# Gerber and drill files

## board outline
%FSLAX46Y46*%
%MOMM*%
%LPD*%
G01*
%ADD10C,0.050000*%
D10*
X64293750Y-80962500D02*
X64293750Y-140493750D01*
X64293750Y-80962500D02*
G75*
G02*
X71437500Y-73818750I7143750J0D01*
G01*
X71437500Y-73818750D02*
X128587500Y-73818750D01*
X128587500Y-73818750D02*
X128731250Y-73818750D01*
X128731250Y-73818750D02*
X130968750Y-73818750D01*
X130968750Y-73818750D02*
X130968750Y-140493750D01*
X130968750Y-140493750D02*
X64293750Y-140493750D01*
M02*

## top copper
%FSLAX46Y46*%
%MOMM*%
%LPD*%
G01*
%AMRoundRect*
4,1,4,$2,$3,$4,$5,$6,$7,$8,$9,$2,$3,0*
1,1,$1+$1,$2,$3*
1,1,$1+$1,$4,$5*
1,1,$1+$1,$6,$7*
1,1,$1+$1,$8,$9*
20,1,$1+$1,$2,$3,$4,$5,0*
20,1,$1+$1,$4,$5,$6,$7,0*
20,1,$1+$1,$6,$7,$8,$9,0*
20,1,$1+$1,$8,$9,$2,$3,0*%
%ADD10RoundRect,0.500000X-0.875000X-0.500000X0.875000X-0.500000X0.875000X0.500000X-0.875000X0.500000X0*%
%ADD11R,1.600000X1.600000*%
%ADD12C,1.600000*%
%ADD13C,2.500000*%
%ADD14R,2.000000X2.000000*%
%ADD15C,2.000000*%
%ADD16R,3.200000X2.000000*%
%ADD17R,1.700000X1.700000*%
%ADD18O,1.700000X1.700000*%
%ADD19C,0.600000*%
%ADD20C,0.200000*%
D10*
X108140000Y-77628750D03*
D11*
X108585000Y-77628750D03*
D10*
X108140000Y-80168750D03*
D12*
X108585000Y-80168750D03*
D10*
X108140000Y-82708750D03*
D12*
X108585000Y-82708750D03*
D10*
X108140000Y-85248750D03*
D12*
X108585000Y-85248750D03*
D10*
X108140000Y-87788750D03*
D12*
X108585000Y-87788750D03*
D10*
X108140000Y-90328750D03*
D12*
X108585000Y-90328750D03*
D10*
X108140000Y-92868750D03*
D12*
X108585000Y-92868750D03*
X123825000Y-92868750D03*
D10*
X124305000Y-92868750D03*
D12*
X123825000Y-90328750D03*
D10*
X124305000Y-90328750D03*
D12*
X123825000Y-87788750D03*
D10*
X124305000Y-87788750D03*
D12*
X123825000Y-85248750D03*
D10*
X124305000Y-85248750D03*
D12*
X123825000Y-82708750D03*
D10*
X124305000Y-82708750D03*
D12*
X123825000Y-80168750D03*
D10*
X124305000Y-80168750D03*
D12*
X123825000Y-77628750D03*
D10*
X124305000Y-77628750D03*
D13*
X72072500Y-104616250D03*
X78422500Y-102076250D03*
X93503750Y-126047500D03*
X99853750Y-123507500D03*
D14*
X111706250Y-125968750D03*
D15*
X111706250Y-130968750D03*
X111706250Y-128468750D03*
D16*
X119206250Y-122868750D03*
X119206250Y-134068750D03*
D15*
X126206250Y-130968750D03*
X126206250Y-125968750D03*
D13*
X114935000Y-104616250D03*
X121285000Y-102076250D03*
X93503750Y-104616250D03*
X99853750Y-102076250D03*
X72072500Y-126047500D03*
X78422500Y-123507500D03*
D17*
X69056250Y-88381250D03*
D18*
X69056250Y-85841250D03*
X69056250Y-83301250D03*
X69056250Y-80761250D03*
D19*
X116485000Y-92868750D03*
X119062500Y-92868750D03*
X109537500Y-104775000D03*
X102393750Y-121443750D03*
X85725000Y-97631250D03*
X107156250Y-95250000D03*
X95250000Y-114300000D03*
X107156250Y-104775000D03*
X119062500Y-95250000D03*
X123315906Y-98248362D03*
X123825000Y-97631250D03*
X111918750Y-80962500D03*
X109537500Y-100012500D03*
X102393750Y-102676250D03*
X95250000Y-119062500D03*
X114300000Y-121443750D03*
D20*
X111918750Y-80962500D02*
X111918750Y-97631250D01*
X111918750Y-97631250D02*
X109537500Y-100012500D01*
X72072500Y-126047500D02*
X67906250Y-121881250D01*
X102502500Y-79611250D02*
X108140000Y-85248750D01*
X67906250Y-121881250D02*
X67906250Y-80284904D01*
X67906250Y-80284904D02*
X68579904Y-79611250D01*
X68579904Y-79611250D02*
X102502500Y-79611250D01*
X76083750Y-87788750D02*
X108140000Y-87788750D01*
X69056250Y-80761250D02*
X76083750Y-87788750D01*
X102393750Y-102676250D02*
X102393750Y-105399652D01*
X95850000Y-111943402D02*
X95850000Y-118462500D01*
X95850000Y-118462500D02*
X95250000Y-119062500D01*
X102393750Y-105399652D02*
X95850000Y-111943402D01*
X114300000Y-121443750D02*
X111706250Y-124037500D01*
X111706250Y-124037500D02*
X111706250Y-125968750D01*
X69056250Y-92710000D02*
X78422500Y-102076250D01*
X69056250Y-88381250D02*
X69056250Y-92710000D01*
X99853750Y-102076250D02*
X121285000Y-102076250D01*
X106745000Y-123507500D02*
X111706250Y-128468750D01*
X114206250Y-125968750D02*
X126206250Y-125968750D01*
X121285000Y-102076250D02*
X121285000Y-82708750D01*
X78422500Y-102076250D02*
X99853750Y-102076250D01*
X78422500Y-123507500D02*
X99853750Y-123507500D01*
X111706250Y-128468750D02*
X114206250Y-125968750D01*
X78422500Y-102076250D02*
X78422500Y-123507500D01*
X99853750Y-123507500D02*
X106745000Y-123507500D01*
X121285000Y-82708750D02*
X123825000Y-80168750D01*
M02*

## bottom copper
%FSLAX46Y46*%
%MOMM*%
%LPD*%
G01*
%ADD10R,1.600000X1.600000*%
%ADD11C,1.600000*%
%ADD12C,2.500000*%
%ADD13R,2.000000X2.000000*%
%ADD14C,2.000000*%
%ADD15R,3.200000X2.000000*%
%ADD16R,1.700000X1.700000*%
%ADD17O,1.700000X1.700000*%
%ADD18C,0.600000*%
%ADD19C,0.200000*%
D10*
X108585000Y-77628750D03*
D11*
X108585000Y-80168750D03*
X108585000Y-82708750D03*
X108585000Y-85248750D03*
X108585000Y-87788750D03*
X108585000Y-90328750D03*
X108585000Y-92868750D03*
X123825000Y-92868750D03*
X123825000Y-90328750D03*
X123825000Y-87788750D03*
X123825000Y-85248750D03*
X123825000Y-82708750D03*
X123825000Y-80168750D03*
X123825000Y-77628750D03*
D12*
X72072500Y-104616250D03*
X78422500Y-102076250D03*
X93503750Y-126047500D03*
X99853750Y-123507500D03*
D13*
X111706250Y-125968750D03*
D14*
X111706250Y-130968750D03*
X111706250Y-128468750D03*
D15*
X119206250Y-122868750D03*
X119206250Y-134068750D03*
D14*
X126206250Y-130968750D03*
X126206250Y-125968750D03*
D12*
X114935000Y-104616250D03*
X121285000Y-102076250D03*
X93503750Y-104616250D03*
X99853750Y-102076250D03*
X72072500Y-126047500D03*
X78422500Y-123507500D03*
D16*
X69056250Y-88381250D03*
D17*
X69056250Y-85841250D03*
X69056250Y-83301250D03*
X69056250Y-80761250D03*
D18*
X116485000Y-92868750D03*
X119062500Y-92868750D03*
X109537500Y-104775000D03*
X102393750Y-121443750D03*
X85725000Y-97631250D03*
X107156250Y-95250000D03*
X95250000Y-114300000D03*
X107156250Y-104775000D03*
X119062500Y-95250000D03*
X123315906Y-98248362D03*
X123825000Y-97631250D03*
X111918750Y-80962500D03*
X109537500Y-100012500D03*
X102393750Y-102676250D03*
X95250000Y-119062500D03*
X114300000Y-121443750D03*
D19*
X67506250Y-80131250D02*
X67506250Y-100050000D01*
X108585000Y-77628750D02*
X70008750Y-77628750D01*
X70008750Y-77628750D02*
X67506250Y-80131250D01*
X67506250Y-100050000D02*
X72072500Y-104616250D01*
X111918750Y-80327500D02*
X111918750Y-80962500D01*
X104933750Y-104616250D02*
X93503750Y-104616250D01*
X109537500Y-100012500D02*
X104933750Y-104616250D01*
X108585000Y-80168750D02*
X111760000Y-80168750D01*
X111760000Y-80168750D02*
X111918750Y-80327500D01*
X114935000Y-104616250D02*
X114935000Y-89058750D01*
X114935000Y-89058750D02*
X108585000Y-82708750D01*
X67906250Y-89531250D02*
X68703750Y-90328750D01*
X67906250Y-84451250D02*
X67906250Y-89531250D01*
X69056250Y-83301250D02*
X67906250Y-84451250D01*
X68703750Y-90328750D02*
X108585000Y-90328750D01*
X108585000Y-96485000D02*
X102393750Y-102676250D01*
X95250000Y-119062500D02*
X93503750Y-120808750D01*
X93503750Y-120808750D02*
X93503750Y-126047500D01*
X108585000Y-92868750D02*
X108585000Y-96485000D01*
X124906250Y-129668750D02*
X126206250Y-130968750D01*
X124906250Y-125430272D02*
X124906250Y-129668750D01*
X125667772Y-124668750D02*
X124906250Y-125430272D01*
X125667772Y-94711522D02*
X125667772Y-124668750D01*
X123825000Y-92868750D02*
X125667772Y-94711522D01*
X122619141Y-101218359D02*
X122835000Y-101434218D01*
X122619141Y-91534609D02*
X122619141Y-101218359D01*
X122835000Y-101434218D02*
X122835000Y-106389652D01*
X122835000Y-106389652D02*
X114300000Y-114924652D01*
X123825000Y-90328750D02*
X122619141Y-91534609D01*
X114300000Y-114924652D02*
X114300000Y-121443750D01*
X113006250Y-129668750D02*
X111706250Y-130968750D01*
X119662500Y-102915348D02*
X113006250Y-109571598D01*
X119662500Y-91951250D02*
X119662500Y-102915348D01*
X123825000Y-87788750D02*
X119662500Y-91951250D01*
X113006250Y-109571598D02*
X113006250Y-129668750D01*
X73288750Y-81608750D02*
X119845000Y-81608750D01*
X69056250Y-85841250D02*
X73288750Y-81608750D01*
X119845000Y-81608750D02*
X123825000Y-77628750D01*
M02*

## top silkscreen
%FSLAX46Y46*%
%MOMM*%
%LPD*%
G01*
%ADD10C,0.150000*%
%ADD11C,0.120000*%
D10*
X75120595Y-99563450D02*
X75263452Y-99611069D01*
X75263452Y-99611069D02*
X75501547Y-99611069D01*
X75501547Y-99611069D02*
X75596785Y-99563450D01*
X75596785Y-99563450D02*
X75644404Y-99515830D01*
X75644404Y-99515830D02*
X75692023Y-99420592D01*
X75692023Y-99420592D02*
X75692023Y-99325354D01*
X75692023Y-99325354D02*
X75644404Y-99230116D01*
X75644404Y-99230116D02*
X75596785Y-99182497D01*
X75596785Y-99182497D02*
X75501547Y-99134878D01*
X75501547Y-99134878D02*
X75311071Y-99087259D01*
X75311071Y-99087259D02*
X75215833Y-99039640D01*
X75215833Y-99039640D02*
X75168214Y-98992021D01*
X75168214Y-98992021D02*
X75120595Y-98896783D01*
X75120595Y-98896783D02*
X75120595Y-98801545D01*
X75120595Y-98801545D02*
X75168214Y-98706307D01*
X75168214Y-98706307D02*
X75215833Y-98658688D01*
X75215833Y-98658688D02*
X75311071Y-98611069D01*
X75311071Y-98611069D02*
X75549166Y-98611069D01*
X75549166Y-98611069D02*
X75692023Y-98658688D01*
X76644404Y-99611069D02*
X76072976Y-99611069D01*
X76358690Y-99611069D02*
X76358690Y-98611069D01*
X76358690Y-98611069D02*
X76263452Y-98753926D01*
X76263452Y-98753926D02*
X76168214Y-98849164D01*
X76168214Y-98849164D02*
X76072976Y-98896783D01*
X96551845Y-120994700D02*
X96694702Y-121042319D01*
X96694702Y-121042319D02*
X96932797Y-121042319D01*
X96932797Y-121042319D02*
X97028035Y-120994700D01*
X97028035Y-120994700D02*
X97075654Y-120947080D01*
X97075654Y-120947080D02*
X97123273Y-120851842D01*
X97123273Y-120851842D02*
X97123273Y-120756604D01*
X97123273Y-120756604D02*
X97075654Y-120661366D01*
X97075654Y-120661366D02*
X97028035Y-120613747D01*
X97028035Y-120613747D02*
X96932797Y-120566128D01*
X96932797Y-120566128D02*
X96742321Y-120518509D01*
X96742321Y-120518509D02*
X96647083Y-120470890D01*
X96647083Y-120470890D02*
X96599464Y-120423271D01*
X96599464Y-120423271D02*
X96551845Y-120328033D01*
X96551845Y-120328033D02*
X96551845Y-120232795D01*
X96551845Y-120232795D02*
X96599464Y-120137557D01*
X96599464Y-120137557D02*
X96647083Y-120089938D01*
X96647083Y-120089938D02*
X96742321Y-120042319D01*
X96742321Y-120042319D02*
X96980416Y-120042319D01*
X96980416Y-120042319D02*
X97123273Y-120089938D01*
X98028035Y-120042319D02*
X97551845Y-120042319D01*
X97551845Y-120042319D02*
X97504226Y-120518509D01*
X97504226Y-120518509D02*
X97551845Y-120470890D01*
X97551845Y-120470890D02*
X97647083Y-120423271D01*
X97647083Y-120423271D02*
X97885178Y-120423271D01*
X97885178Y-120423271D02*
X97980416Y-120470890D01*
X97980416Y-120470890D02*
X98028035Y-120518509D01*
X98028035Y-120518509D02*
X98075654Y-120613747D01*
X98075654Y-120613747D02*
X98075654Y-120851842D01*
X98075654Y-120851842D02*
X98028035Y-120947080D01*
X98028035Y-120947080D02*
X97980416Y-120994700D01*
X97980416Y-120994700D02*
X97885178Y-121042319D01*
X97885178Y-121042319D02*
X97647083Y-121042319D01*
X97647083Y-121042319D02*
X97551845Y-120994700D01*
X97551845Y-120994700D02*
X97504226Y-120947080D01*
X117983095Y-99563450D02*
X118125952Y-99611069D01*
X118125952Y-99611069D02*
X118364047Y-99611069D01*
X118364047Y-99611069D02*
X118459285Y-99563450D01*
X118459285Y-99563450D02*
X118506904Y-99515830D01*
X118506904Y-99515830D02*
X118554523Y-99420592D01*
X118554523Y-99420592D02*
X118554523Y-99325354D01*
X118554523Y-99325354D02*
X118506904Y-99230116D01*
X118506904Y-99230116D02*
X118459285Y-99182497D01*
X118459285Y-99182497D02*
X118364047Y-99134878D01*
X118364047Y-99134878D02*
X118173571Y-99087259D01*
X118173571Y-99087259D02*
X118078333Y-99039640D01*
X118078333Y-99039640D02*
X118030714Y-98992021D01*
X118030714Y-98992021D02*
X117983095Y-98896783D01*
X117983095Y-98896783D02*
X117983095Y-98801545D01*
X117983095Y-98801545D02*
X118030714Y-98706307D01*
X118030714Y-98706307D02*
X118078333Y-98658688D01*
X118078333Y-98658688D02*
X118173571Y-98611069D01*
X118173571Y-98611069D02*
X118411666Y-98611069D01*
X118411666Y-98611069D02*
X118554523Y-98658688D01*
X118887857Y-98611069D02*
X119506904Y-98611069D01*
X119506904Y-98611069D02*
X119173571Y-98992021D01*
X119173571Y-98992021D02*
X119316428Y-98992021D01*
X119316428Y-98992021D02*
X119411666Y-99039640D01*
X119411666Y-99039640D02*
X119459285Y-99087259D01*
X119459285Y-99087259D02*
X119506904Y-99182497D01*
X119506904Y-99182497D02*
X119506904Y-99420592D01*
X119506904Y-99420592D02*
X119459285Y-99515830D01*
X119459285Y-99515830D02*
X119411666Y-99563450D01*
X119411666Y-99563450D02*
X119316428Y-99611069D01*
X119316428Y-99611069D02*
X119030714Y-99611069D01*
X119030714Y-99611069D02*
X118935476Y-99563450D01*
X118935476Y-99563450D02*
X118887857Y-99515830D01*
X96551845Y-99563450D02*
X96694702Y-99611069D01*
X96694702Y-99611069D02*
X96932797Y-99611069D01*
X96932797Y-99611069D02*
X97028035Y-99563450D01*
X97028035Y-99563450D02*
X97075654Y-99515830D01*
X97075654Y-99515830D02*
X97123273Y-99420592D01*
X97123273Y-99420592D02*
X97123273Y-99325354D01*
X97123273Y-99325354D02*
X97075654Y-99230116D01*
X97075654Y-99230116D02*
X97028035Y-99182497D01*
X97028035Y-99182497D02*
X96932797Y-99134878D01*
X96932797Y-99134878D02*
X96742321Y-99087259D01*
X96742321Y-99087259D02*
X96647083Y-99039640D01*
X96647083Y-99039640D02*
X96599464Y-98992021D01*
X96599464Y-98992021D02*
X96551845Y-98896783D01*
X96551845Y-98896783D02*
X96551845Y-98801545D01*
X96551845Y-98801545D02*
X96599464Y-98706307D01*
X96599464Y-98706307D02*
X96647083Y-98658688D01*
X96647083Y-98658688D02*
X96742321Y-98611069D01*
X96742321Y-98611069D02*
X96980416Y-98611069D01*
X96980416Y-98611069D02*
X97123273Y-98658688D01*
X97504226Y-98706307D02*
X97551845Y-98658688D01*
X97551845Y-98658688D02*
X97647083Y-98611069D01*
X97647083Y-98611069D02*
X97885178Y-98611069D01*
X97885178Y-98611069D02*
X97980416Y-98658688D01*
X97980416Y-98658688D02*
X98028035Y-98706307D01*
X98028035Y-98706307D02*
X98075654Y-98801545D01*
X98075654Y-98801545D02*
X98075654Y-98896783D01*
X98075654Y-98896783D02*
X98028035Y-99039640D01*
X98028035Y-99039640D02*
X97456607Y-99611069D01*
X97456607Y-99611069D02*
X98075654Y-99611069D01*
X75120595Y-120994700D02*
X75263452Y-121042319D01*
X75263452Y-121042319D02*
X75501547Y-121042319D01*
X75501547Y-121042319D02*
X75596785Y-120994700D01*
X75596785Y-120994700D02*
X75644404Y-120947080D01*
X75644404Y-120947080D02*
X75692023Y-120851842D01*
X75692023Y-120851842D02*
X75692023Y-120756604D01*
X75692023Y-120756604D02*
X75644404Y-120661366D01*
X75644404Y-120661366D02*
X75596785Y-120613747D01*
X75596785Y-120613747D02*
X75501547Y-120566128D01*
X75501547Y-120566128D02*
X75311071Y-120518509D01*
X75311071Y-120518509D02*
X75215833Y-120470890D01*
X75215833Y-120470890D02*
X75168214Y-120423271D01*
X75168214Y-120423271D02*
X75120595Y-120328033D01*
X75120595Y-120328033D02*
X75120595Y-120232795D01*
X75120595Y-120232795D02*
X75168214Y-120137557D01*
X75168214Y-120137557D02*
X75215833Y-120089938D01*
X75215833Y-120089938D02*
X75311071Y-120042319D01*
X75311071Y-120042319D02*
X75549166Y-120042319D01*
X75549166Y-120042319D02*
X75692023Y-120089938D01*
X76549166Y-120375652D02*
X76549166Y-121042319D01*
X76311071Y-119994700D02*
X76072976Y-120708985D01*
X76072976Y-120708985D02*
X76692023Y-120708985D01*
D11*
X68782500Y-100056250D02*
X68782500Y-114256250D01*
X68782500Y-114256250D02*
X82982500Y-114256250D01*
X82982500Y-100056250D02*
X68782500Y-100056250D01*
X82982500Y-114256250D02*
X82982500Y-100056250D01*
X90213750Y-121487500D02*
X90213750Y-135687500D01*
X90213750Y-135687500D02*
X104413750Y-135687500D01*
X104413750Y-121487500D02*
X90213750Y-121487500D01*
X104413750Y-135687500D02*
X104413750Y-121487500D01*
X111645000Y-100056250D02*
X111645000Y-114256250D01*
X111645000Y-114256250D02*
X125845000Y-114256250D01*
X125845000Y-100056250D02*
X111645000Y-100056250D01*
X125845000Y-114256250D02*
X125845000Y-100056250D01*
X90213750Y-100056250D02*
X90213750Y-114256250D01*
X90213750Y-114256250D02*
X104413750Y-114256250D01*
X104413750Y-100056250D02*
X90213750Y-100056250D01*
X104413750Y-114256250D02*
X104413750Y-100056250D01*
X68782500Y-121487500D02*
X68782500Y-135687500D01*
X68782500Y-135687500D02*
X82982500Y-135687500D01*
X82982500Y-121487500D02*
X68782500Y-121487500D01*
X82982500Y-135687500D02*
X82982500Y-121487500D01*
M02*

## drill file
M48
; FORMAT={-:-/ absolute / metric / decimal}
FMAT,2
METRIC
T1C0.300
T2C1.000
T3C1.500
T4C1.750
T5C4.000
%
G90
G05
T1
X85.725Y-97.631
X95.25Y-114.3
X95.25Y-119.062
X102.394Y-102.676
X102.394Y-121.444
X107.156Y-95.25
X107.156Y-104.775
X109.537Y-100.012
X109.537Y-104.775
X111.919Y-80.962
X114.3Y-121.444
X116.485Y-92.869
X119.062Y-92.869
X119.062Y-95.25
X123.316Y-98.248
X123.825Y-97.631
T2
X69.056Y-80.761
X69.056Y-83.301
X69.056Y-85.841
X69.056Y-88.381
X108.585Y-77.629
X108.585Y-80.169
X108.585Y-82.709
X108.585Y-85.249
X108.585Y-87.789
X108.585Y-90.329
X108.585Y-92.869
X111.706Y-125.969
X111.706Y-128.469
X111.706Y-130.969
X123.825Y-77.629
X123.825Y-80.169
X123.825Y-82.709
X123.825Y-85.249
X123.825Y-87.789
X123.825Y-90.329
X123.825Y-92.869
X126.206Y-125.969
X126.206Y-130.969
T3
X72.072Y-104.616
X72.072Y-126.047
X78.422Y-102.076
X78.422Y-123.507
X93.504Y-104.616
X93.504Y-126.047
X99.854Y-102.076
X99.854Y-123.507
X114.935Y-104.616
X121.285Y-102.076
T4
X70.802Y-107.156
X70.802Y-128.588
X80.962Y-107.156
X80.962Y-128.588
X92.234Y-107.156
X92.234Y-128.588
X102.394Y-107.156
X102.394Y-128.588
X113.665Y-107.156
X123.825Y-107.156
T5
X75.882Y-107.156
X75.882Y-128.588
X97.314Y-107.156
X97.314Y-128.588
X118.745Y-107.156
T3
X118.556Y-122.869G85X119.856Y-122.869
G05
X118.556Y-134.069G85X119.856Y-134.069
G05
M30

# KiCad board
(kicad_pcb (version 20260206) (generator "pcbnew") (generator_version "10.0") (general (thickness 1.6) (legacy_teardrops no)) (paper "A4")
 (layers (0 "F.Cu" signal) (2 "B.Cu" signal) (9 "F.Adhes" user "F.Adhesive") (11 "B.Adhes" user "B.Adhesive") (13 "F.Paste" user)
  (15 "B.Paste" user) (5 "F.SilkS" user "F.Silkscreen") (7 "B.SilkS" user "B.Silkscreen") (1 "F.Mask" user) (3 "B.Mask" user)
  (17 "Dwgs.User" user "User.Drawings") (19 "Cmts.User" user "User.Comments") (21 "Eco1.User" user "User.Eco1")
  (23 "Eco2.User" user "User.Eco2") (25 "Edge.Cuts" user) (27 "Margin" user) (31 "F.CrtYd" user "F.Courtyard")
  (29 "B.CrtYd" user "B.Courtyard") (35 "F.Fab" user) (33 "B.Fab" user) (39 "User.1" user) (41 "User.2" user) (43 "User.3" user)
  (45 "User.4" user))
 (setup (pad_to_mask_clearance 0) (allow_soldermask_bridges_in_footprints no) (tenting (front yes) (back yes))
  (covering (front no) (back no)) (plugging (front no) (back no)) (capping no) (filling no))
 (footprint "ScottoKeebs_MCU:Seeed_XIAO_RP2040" (layer "F.Cu") (at 116.205 85.24875)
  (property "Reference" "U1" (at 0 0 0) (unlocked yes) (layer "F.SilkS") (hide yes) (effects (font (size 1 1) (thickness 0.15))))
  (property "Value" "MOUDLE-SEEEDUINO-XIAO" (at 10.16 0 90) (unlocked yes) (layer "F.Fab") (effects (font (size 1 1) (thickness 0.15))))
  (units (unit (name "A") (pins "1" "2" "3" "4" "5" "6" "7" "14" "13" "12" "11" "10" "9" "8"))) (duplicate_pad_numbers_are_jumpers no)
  (pad "1" smd roundrect (at -8.065 -7.62) (size 2.75 2) (layers "F.Cu" "F.Mask" "F.Paste") (roundrect_rratio 0.25) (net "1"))
  (pad "1" thru_hole rect (at -7.62 -7.62 90) (size 1.6 1.6) (drill 1) (layers "*.Cu" "*.Mask") (remove_unused_layers no) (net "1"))
  (pad "2" smd roundrect (at -8.065 -5.08) (size 2.75 2) (layers "F.Cu" "F.Mask" "F.Paste") (roundrect_rratio 0.25) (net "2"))
  (pad "2" thru_hole circle (at -7.62 -5.08 90) (size 1.6 1.6) (drill 1) (layers "*.Cu" "*.Mask") (remove_unused_layers no) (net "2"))
  (pad "3" smd roundrect (at -8.065 -2.54) (size 2.75 2) (layers "F.Cu" "F.Mask" "F.Paste") (roundrect_rratio 0.25) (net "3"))
  (pad "3" thru_hole circle (at -7.62 -2.54 90) (size 1.6 1.6) (drill 1) (layers "*.Cu" "*.Mask") (remove_unused_layers no) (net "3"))
  (pad "4" smd roundrect (at -8.065 0) (size 2.75 2) (layers "F.Cu" "F.Mask" "F.Paste") (roundrect_rratio 0.25) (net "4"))
  (pad "4" thru_hole circle (at -7.62 0 90) (size 1.6 1.6) (drill 1) (layers "*.Cu" "*.Mask") (remove_unused_layers no) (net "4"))
  (pad "5" smd roundrect (at -8.065 2.54) (size 2.75 2) (layers "F.Cu" "F.Mask" "F.Paste") (roundrect_rratio 0.25) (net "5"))
  (pad "5" thru_hole circle (at -7.62 2.54 90) (size 1.6 1.6) (drill 1) (layers "*.Cu" "*.Mask") (remove_unused_layers no) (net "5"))
  (pad "6" smd roundrect (at -8.065 5.08) (size 2.75 2) (layers "F.Cu" "F.Mask" "F.Paste") (roundrect_rratio 0.25) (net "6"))
  (pad "6" thru_hole circle (at -7.62 5.08 90) (size 1.6 1.6) (drill 1) (layers "*.Cu" "*.Mask") (remove_unused_layers no) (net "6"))
  (pad "7" smd roundrect (at -8.065 7.62) (size 2.75 2) (layers "F.Cu" "F.Mask" "F.Paste") (roundrect_rratio 0.25) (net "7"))
  (pad "7" thru_hole circle (at -7.62 7.62 90) (size 1.6 1.6) (drill 1) (layers "*.Cu" "*.Mask") (remove_unused_layers no) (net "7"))
  (pad "8" thru_hole circle (at 7.62 7.62 90) (size 1.6 1.6) (drill 1) (layers "*.Cu" "*.Mask") (remove_unused_layers no) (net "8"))
  (pad "8" smd roundrect (at 8.1 7.62) (size 2.75 2) (layers "F.Cu" "F.Mask" "F.Paste") (roundrect_rratio 0.25) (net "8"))
  (pad "9" thru_hole circle (at 7.62 5.08 90) (size 1.6 1.6) (drill 1) (layers "*.Cu" "*.Mask") (remove_unused_layers no) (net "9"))
  (pad "9" smd roundrect (at 8.1 5.08) (size 2.75 2) (layers "F.Cu" "F.Mask" "F.Paste") (roundrect_rratio 0.25) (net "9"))
  (pad "10" thru_hole circle (at 7.62 2.54 90) (size 1.6 1.6) (drill 1) (layers "*.Cu" "*.Mask") (remove_unused_layers no) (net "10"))
  (pad "10" smd roundrect (at 8.1 2.54) (size 2.75 2) (layers "F.Cu" "F.Mask" "F.Paste") (roundrect_rratio 0.25) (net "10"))
  (pad "11" thru_hole circle (at 7.62 0 90) (size 1.6 1.6) (drill 1) (layers "*.Cu" "*.Mask") (remove_unused_layers no) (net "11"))
  (pad "11" smd roundrect (at 8.1 0) (size 2.75 2) (layers "F.Cu" "F.Mask" "F.Paste") (roundrect_rratio 0.25) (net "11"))
  (pad "12" thru_hole circle (at 7.62 -2.54 90) (size 1.6 1.6) (drill 1) (layers "*.Cu" "*.Mask") (remove_unused_layers no) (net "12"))
  (pad "12" smd roundrect (at 8.1 -2.54) (size 2.75 2) (layers "F.Cu" "F.Mask" "F.Paste") (roundrect_rratio 0.25) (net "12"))
  (pad "13" thru_hole circle (at 7.62 -5.08 90) (size 1.6 1.6) (drill 1) (layers "*.Cu" "*.Mask") (remove_unused_layers no) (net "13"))
  (pad "13" smd roundrect (at 8.1 -5.08) (size 2.75 2) (layers "F.Cu" "F.Mask" "F.Paste") (roundrect_rratio 0.25) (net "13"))
  (pad "14" thru_hole circle (at 7.62 -7.62 90) (size 1.6 1.6) (drill 1) (layers "*.Cu" "*.Mask") (remove_unused_layers no) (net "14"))
  (pad "14" smd roundrect (at 8.1 -7.62) (size 2.75 2) (layers "F.Cu" "F.Mask" "F.Paste") (roundrect_rratio 0.25) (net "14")))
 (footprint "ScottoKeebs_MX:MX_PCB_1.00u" (layer "F.Cu") (at 75.8825 107.15625)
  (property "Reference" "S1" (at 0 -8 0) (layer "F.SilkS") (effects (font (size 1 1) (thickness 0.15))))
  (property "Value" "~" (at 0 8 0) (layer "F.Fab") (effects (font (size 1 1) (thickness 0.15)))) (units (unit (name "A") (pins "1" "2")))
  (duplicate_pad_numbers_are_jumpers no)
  (fp_line (start -7.1 -7.1) (end -7.1 7.1) (stroke (width 0.12) (type solid)) (layer "F.SilkS"))
  (fp_line (start -7.1 7.1) (end 7.1 7.1) (stroke (width 0.12) (type solid)) (layer "F.SilkS"))
  (fp_line (start 7.1 -7.1) (end -7.1 -7.1) (stroke (width 0.12) (type solid)) (layer "F.SilkS"))
  (fp_line (start 7.1 7.1) (end 7.1 -7.1) (stroke (width 0.12) (type solid)) (layer "F.SilkS"))
  (pad "" np_thru_hole circle (at -5.08 0) (size 1.75 1.75) (drill 1.75) (layers "*.Cu" "*.Mask"))
  (pad "" np_thru_hole circle (at 0 0) (size 4 4) (drill 4) (layers "*.Cu" "*.Mask"))
  (pad "" np_thru_hole circle (at 5.08 0) (size 1.75 1.75) (drill 1.75) (layers "*.Cu" "*.Mask"))
  (pad "1" thru_hole circle (at -3.81 -2.54) (size 2.5 2.5) (drill 1.5) (layers "*.Cu" "*.Mask") (remove_unused_layers no) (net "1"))
  (pad "2" thru_hole circle (at 2.54 -5.08) (size 2.5 2.5) (drill 1.5) (layers "*.Cu" "*.Mask") (remove_unused_layers no) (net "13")))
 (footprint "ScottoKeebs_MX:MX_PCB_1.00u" (layer "F.Cu") (at 97.31375 128.5875)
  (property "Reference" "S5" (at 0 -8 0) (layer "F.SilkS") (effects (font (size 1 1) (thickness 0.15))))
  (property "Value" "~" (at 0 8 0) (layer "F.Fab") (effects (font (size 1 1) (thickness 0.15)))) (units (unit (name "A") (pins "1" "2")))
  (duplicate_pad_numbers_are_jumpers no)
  (fp_line (start -7.1 -7.1) (end -7.1 7.1) (stroke (width 0.12) (type solid)) (layer "F.SilkS"))
  (fp_line (start -7.1 7.1) (end 7.1 7.1) (stroke (width 0.12) (type solid)) (layer "F.SilkS"))
  (fp_line (start 7.1 -7.1) (end -7.1 -7.1) (stroke (width 0.12) (type solid)) (layer "F.SilkS"))
  (fp_line (start 7.1 7.1) (end 7.1 -7.1) (stroke (width 0.12) (type solid)) (layer "F.SilkS"))
  (pad "" np_thru_hole circle (at -5.08 0) (size 1.75 1.75) (drill 1.75) (layers "*.Cu" "*.Mask"))
  (pad "" np_thru_hole circle (at 0 0) (size 4 4) (drill 4) (layers "*.Cu" "*.Mask"))
  (pad "" np_thru_hole circle (at 5.08 0) (size 1.75 1.75) (drill 1.75) (layers "*.Cu" "*.Mask"))
  (pad "1" thru_hole circle (at -3.81 -2.54) (size 2.5 2.5) (drill 1.5) (layers "*.Cu" "*.Mask") (remove_unused_layers no) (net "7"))
  (pad "2" thru_hole circle (at 2.54 -5.08) (size 2.5 2.5) (drill 1.5) (layers "*.Cu" "*.Mask") (remove_unused_layers no) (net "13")))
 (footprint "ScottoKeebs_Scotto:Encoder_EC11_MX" (layer "F.Cu") (at 119.20625 128.46875)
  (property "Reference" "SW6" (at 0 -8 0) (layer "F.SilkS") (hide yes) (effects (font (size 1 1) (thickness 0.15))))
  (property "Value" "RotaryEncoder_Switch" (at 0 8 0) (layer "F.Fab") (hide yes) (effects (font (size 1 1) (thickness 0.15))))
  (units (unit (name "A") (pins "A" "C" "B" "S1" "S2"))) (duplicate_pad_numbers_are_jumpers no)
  (pad "A" thru_hole rect (at -7.5 -2.5) (size 2 2) (drill 1) (layers "*.Cu" "*.Mask") (remove_unused_layers no) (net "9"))
  (pad "B" thru_hole circle (at -7.5 2.5) (size 2 2) (drill 1) (layers "*.Cu" "*.Mask") (remove_unused_layers no) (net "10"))
  (pad "C" thru_hole circle (at -7.5 0) (size 2 2) (drill 1) (layers "*.Cu" "*.Mask") (remove_unused_layers no) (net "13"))
  (pad "MP" thru_hole rect (at 0 -5.6) (size 3.2 2) (drill oval 2.8 1.5) (layers "*.Cu" "*.Mask") (remove_unused_layers no))
  (pad "MP" thru_hole rect (at 0 5.6) (size 3.2 2) (drill oval 2.8 1.5) (layers "*.Cu" "*.Mask") (remove_unused_layers no))
  (pad "S1" thru_hole circle (at 7 2.5) (size 2 2) (drill 1) (layers "*.Cu" "*.Mask") (remove_unused_layers no) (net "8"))
  (pad "S2" thru_hole circle (at 7 -2.5) (size 2 2) (drill 1) (layers "*.Cu" "*.Mask") (remove_unused_layers no) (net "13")))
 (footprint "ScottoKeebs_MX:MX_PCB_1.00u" (layer "F.Cu") (at 118.745 107.15625)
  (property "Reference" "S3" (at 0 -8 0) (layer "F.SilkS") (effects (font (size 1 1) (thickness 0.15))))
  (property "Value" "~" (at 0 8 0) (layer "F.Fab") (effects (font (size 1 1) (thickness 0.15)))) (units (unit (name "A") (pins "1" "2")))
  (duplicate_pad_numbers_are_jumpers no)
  (fp_line (start -7.1 -7.1) (end -7.1 7.1) (stroke (width 0.12) (type solid)) (layer "F.SilkS"))
  (fp_line (start -7.1 7.1) (end 7.1 7.1) (stroke (width 0.12) (type solid)) (layer "F.SilkS"))
  (fp_line (start 7.1 -7.1) (end -7.1 -7.1) (stroke (width 0.12) (type solid)) (layer "F.SilkS"))
  (fp_line (start 7.1 7.1) (end 7.1 -7.1) (stroke (width 0.12) (type solid)) (layer "F.SilkS"))
  (pad "" np_thru_hole circle (at -5.08 0) (size 1.75 1.75) (drill 1.75) (layers "*.Cu" "*.Mask"))
  (pad "" np_thru_hole circle (at 0 0) (size 4 4) (drill 4) (layers "*.Cu" "*.Mask"))
  (pad "" np_thru_hole circle (at 5.08 0) (size 1.75 1.75) (drill 1.75) (layers "*.Cu" "*.Mask"))
  (pad "1" thru_hole circle (at -3.81 -2.54) (size 2.5 2.5) (drill 1.5) (layers "*.Cu" "*.Mask") (remove_unused_layers no) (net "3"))
  (pad "2" thru_hole circle (at 2.54 -5.08) (size 2.5 2.5) (drill 1.5) (layers "*.Cu" "*.Mask") (remove_unused_layers no) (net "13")))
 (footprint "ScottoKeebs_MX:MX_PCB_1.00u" (layer "F.Cu") (at 97.31375 107.15625)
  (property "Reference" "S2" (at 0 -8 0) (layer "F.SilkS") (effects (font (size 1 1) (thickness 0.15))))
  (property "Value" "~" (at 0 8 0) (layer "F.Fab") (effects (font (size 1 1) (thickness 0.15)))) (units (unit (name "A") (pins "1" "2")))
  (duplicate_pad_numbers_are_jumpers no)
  (fp_line (start -7.1 -7.1) (end -7.1 7.1) (stroke (width 0.12) (type solid)) (layer "F.SilkS"))
  (fp_line (start -7.1 7.1) (end 7.1 7.1) (stroke (width 0.12) (type solid)) (layer "F.SilkS"))
  (fp_line (start 7.1 -7.1) (end -7.1 -7.1) (stroke (width 0.12) (type solid)) (layer "F.SilkS"))
  (fp_line (start 7.1 7.1) (end 7.1 -7.1) (stroke (width 0.12) (type solid)) (layer "F.SilkS"))
  (pad "" np_thru_hole circle (at -5.08 0) (size 1.75 1.75) (drill 1.75) (layers "*.Cu" "*.Mask"))
  (pad "" np_thru_hole circle (at 0 0) (size 4 4) (drill 4) (layers "*.Cu" "*.Mask"))
  (pad "" np_thru_hole circle (at 5.08 0) (size 1.75 1.75) (drill 1.75) (layers "*.Cu" "*.Mask"))
  (pad "1" thru_hole circle (at -3.81 -2.54) (size 2.5 2.5) (drill 1.5) (layers "*.Cu" "*.Mask") (remove_unused_layers no) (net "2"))
  (pad "2" thru_hole circle (at 2.54 -5.08) (size 2.5 2.5) (drill 1.5) (layers "*.Cu" "*.Mask") (remove_unused_layers no) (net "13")))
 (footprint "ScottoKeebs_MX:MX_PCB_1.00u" (layer "F.Cu") (at 75.8825 128.5875)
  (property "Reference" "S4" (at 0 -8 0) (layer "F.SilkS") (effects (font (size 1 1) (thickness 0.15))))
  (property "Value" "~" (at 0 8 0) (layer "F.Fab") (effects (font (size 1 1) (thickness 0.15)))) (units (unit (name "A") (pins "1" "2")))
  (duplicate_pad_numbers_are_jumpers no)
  (fp_line (start -7.1 -7.1) (end -7.1 7.1) (stroke (width 0.12) (type solid)) (layer "F.SilkS"))
  (fp_line (start -7.1 7.1) (end 7.1 7.1) (stroke (width 0.12) (type solid)) (layer "F.SilkS"))
  (fp_line (start 7.1 -7.1) (end -7.1 -7.1) (stroke (width 0.12) (type solid)) (layer "F.SilkS"))
  (fp_line (start 7.1 7.1) (end 7.1 -7.1) (stroke (width 0.12) (type solid)) (layer "F.SilkS"))
  (pad "" np_thru_hole circle (at -5.08 0) (size 1.75 1.75) (drill 1.75) (layers "*.Cu" "*.Mask"))
  (pad "" np_thru_hole circle (at 0 0) (size 4 4) (drill 4) (layers "*.Cu" "*.Mask"))
  (pad "" np_thru_hole circle (at 5.08 0) (size 1.75 1.75) (drill 1.75) (layers "*.Cu" "*.Mask"))
  (pad "1" thru_hole circle (at -3.81 -2.54) (size 2.5 2.5) (drill 1.5) (layers "*.Cu" "*.Mask") (remove_unused_layers no) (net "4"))
  (pad "2" thru_hole circle (at 2.54 -5.08) (size 2.5 2.5) (drill 1.5) (layers "*.Cu" "*.Mask") (remove_unused_layers no) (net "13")))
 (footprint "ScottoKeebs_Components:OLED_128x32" (layer "F.Cu") (at 67.45625 78.58125)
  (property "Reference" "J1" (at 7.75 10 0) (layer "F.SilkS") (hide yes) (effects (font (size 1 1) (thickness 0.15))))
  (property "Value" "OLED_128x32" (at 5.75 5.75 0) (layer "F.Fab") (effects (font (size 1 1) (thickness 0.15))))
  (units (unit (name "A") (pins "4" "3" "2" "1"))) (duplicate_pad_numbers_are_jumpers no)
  (pad "1" thru_hole rect (at 1.6 9.8 180) (size 1.7 1.7) (drill 1) (layers "*.Cu" "*.Mask") (remove_unused_layers no) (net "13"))
  (pad "2" thru_hole oval (at 1.6 7.26 180) (size 1.7 1.7) (drill 1) (layers "*.Cu" "*.Mask") (remove_unused_layers no) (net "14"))
  (pad "3" thru_hole oval (at 1.6 4.72 180) (size 1.7 1.7) (drill 1) (layers "*.Cu" "*.Mask") (remove_unused_layers no) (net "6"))
  (pad "4" thru_hole oval (at 1.6 2.18 180) (size 1.7 1.7) (drill 1) (layers "*.Cu" "*.Mask") (remove_unused_layers no) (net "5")))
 (gr_line (start 64.29375 80.9625) (end 64.29375 140.49375) (stroke (width 0.05) (type default)) (layer "Edge.Cuts"))
 (gr_arc (start 64.29375 80.9625) (mid 66.386106 75.911106) (end 71.4375 73.81875) (stroke (width 0.05) (type default)) (layer "Edge.Cuts"))
 (gr_line (start 71.4375 73.81875) (end 128.5875 73.81875) (stroke (width 0.05) (type default)) (layer "Edge.Cuts"))
 (gr_line (start 128.5875 73.81875) (end 128.73125 73.81875) (stroke (width 0.05) (type default)) (layer "Edge.Cuts"))
 (gr_line (start 128.73125 73.81875) (end 130.96875 73.81875) (stroke (width 0.05) (type default)) (layer "Edge.Cuts"))
 (gr_line (start 130.96875 73.81875) (end 130.96875 140.49375) (stroke (width 0.05) (type default)) (layer "Edge.Cuts"))
 (gr_line (start 130.96875 140.49375) (end 64.29375 140.49375) (stroke (width 0.05) (type default)) (layer "Edge.Cuts"))
 (via (at 116.485 92.86875) (size 0.6) (drill 0.3) (layers "F.Cu" "B.Cu") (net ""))
 (via (at 119.0625 92.86875) (size 0.6) (drill 0.3) (layers "F.Cu" "B.Cu") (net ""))
 (via (at 109.5375 104.775) (size 0.6) (drill 0.3) (layers "F.Cu" "B.Cu") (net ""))
 (via (at 102.39375 121.44375) (size 0.6) (drill 0.3) (layers "F.Cu" "B.Cu") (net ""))
 (via (at 85.725 97.63125) (size 0.6) (drill 0.3) (layers "F.Cu" "B.Cu") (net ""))
 (via (at 107.15625 95.25) (size 0.6) (drill 0.3) (layers "F.Cu" "B.Cu") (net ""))
 (via (at 95.25 114.3) (size 0.6) (drill 0.3) (layers "F.Cu" "B.Cu") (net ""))
 (via (at 107.15625 104.775) (size 0.6) (drill 0.3) (layers "F.Cu" "B.Cu") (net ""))
 (via (at 119.0625 95.25) (size 0.6) (drill 0.3) (layers "F.Cu" "B.Cu") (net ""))
 (via (at 123.315906 98.248362) (size 0.6) (drill 0.3) (layers "F.Cu" "B.Cu") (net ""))
 (via (at 123.825 97.63125) (size 0.6) (drill 0.3) (layers "F.Cu" "B.Cu") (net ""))
 (segment (start 67.50625 80.13125) (end 67.50625 100.05) (width 0.2) (layer "B.Cu") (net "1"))
 (segment (start 108.585 77.62875) (end 70.00875 77.62875) (width 0.2) (layer "B.Cu") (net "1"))
 (segment (start 70.00875 77.62875) (end 67.50625 80.13125) (width 0.2) (layer "B.Cu") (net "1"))
 (segment (start 67.50625 100.05) (end 72.0725 104.61625) (width 0.2) (layer "B.Cu") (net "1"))
 (segment (start 111.91875 80.9625) (end 111.91875 97.63125) (width 0.2) (layer "F.Cu") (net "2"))
 (segment (start 111.91875 97.63125) (end 109.5375 100.0125) (width 0.2) (layer "F.Cu") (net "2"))
 (via (at 111.91875 80.9625) (size 0.6) (drill 0.3) (layers "F.Cu" "B.Cu") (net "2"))
 (via (at 109.5375 100.0125) (size 0.6) (drill 0.3) (layers "F.Cu" "B.Cu") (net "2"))
 (segment (start 111.91875 80.3275) (end 111.91875 80.9625) (width 0.2) (layer "B.Cu") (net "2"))
 (segment (start 104.93375 104.61625) (end 93.50375 104.61625) (width 0.2) (layer "B.Cu") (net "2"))
 (segment (start 109.5375 100.0125) (end 104.93375 104.61625) (width 0.2) (layer "B.Cu") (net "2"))
 (segment (start 108.585 80.16875) (end 111.76 80.16875) (width 0.2) (layer "B.Cu") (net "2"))
 (segment (start 111.76 80.16875) (end 111.91875 80.3275) (width 0.2) (layer "B.Cu") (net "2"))
 (segment (start 114.935 104.61625) (end 114.935 89.05875) (width 0.2) (layer "B.Cu") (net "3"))
 (segment (start 114.935 89.05875) (end 108.585 82.70875) (width 0.2) (layer "B.Cu") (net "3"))
 (segment (start 72.0725 126.0475) (end 67.90625 121.88125) (width 0.2) (layer "F.Cu") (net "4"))
 (segment (start 102.5025 79.61125) (end 108.14 85.24875) (width 0.2) (layer "F.Cu") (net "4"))
 (segment (start 67.90625 121.88125) (end 67.90625 80.284904) (width 0.2) (layer "F.Cu") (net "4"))
 (segment (start 67.90625 80.284904) (end 68.579904 79.61125) (width 0.2) (layer "F.Cu") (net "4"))
 (segment (start 68.579904 79.61125) (end 102.5025 79.61125) (width 0.2) (layer "F.Cu") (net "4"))
 (segment (start 76.08375 87.78875) (end 108.14 87.78875) (width 0.2) (layer "F.Cu") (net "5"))
 (segment (start 69.05625 80.76125) (end 76.08375 87.78875) (width 0.2) (layer "F.Cu") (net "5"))
 (segment (start 67.90625 89.53125) (end 68.70375 90.32875) (width 0.2) (layer "B.Cu") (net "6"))
 (segment (start 67.90625 84.45125) (end 67.90625 89.53125) (width 0.2) (layer "B.Cu") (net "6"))
 (segment (start 69.05625 83.30125) (end 67.90625 84.45125) (width 0.2) (layer "B.Cu") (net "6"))
 (segment (start 68.70375 90.32875) (end 108.585 90.32875) (width 0.2) (layer "B.Cu") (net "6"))
 (segment (start 102.39375 102.67625) (end 102.39375 105.399652) (width 0.2) (layer "F.Cu") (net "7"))
 (segment (start 95.85 111.943402) (end 95.85 118.4625) (width 0.2) (layer "F.Cu") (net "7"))
 (segment (start 95.85 118.4625) (end 95.25 119.0625) (width 0.2) (layer "F.Cu") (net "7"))
 (segment (start 102.39375 105.399652) (end 95.85 111.943402) (width 0.2) (layer "F.Cu") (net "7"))
 (via (at 102.39375 102.67625) (size 0.6) (drill 0.3) (layers "F.Cu" "B.Cu") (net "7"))
 (via (at 95.25 119.0625) (size 0.6) (drill 0.3) (layers "F.Cu" "B.Cu") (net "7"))
 (segment (start 108.585 96.485) (end 102.39375 102.67625) (width 0.2) (layer "B.Cu") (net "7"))
 (segment (start 95.25 119.0625) (end 93.50375 120.80875) (width 0.2) (layer "B.Cu") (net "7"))
 (segment (start 93.50375 120.80875) (end 93.50375 126.0475) (width 0.2) (layer "B.Cu") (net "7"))
 (segment (start 108.585 92.86875) (end 108.585 96.485) (width 0.2) (layer "B.Cu") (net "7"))
 (segment (start 124.90625 129.66875) (end 126.20625 130.96875) (width 0.2) (layer "B.Cu") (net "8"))
 (segment (start 124.90625 125.430272) (end 124.90625 129.66875) (width 0.2) (layer "B.Cu") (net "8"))
 (segment (start 125.667772 124.66875) (end 124.90625 125.430272) (width 0.2) (layer "B.Cu") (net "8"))
 (segment (start 125.667772 94.711522) (end 125.667772 124.66875) (width 0.2) (layer "B.Cu") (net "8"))
 (segment (start 123.825 92.86875) (end 125.667772 94.711522) (width 0.2) (layer "B.Cu") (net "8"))
 (segment (start 114.3 121.44375) (end 111.70625 124.0375) (width 0.2) (layer "F.Cu") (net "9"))
 (segment (start 111.70625 124.0375) (end 111.70625 125.96875) (width 0.2) (layer "F.Cu") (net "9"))
 (via (at 114.3 121.44375) (size 0.6) (drill 0.3) (layers "F.Cu" "B.Cu") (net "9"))
 (segment (start 122.619141 101.218359) (end 122.835 101.434218) (width 0.2) (layer "B.Cu") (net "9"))
 (segment (start 122.619141 91.534609) (end 122.619141 101.218359) (width 0.2) (layer "B.Cu") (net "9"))
 (segment (start 122.835 101.434218) (end 122.835 106.389652) (width 0.2) (layer "B.Cu") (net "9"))
 (segment (start 122.835 106.389652) (end 114.3 114.924652) (width 0.2) (layer "B.Cu") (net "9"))
 (segment (start 123.825 90.32875) (end 122.619141 91.534609) (width 0.2) (layer "B.Cu") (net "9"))
 (segment (start 114.3 114.924652) (end 114.3 121.44375) (width 0.2) (layer "B.Cu") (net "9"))
 (segment (start 113.00625 129.66875) (end 111.70625 130.96875) (width 0.2) (layer "B.Cu") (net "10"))
 (segment (start 119.6625 102.915348) (end 113.00625 109.571598) (width 0.2) (layer "B.Cu") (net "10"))
 (segment (start 119.6625 91.95125) (end 119.6625 102.915348) (width 0.2) (layer "B.Cu") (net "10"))
 (segment (start 123.825 87.78875) (end 119.6625 91.95125) (width 0.2) (layer "B.Cu") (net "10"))
 (segment (start 113.00625 109.571598) (end 113.00625 129.66875) (width 0.2) (layer "B.Cu") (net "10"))
 (segment (start 69.05625 92.71) (end 78.4225 102.07625) (width 0.2) (layer "F.Cu") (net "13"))
 (segment (start 69.05625 88.38125) (end 69.05625 92.71) (width 0.2) (layer "F.Cu") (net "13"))
 (segment (start 99.85375 102.07625) (end 121.285 102.07625) (width 0.2) (layer "F.Cu") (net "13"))
 (segment (start 106.745 123.5075) (end 111.70625 128.46875) (width 0.2) (layer "F.Cu") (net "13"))
 (segment (start 114.20625 125.96875) (end 126.20625 125.96875) (width 0.2) (layer "F.Cu") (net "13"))
 (segment (start 121.285 102.07625) (end 121.285 82.70875) (width 0.2) (layer "F.Cu") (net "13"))
 (segment (start 78.4225 102.07625) (end 99.85375 102.07625) (width 0.2) (layer "F.Cu") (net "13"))
 (segment (start 78.4225 123.5075) (end 99.85375 123.5075) (width 0.2) (layer "F.Cu") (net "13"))
 (segment (start 111.70625 128.46875) (end 114.20625 125.96875) (width 0.2) (layer "F.Cu") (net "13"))
 (segment (start 78.4225 102.07625) (end 78.4225 123.5075) (width 0.2) (layer "F.Cu") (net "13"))
 (segment (start 99.85375 123.5075) (end 106.745 123.5075) (width 0.2) (layer "F.Cu") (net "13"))
 (segment (start 121.285 82.70875) (end 123.825 80.16875) (width 0.2) (layer "F.Cu") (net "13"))
 (segment (start 73.28875 81.60875) (end 119.845 81.60875) (width 0.2) (layer "B.Cu") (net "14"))
 (segment (start 69.05625 85.84125) (end 73.28875 81.60875) (width 0.2) (layer "B.Cu") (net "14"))
 (segment (start 119.845 81.60875) (end 123.825 77.62875) (width 0.2) (layer "B.Cu") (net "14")))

